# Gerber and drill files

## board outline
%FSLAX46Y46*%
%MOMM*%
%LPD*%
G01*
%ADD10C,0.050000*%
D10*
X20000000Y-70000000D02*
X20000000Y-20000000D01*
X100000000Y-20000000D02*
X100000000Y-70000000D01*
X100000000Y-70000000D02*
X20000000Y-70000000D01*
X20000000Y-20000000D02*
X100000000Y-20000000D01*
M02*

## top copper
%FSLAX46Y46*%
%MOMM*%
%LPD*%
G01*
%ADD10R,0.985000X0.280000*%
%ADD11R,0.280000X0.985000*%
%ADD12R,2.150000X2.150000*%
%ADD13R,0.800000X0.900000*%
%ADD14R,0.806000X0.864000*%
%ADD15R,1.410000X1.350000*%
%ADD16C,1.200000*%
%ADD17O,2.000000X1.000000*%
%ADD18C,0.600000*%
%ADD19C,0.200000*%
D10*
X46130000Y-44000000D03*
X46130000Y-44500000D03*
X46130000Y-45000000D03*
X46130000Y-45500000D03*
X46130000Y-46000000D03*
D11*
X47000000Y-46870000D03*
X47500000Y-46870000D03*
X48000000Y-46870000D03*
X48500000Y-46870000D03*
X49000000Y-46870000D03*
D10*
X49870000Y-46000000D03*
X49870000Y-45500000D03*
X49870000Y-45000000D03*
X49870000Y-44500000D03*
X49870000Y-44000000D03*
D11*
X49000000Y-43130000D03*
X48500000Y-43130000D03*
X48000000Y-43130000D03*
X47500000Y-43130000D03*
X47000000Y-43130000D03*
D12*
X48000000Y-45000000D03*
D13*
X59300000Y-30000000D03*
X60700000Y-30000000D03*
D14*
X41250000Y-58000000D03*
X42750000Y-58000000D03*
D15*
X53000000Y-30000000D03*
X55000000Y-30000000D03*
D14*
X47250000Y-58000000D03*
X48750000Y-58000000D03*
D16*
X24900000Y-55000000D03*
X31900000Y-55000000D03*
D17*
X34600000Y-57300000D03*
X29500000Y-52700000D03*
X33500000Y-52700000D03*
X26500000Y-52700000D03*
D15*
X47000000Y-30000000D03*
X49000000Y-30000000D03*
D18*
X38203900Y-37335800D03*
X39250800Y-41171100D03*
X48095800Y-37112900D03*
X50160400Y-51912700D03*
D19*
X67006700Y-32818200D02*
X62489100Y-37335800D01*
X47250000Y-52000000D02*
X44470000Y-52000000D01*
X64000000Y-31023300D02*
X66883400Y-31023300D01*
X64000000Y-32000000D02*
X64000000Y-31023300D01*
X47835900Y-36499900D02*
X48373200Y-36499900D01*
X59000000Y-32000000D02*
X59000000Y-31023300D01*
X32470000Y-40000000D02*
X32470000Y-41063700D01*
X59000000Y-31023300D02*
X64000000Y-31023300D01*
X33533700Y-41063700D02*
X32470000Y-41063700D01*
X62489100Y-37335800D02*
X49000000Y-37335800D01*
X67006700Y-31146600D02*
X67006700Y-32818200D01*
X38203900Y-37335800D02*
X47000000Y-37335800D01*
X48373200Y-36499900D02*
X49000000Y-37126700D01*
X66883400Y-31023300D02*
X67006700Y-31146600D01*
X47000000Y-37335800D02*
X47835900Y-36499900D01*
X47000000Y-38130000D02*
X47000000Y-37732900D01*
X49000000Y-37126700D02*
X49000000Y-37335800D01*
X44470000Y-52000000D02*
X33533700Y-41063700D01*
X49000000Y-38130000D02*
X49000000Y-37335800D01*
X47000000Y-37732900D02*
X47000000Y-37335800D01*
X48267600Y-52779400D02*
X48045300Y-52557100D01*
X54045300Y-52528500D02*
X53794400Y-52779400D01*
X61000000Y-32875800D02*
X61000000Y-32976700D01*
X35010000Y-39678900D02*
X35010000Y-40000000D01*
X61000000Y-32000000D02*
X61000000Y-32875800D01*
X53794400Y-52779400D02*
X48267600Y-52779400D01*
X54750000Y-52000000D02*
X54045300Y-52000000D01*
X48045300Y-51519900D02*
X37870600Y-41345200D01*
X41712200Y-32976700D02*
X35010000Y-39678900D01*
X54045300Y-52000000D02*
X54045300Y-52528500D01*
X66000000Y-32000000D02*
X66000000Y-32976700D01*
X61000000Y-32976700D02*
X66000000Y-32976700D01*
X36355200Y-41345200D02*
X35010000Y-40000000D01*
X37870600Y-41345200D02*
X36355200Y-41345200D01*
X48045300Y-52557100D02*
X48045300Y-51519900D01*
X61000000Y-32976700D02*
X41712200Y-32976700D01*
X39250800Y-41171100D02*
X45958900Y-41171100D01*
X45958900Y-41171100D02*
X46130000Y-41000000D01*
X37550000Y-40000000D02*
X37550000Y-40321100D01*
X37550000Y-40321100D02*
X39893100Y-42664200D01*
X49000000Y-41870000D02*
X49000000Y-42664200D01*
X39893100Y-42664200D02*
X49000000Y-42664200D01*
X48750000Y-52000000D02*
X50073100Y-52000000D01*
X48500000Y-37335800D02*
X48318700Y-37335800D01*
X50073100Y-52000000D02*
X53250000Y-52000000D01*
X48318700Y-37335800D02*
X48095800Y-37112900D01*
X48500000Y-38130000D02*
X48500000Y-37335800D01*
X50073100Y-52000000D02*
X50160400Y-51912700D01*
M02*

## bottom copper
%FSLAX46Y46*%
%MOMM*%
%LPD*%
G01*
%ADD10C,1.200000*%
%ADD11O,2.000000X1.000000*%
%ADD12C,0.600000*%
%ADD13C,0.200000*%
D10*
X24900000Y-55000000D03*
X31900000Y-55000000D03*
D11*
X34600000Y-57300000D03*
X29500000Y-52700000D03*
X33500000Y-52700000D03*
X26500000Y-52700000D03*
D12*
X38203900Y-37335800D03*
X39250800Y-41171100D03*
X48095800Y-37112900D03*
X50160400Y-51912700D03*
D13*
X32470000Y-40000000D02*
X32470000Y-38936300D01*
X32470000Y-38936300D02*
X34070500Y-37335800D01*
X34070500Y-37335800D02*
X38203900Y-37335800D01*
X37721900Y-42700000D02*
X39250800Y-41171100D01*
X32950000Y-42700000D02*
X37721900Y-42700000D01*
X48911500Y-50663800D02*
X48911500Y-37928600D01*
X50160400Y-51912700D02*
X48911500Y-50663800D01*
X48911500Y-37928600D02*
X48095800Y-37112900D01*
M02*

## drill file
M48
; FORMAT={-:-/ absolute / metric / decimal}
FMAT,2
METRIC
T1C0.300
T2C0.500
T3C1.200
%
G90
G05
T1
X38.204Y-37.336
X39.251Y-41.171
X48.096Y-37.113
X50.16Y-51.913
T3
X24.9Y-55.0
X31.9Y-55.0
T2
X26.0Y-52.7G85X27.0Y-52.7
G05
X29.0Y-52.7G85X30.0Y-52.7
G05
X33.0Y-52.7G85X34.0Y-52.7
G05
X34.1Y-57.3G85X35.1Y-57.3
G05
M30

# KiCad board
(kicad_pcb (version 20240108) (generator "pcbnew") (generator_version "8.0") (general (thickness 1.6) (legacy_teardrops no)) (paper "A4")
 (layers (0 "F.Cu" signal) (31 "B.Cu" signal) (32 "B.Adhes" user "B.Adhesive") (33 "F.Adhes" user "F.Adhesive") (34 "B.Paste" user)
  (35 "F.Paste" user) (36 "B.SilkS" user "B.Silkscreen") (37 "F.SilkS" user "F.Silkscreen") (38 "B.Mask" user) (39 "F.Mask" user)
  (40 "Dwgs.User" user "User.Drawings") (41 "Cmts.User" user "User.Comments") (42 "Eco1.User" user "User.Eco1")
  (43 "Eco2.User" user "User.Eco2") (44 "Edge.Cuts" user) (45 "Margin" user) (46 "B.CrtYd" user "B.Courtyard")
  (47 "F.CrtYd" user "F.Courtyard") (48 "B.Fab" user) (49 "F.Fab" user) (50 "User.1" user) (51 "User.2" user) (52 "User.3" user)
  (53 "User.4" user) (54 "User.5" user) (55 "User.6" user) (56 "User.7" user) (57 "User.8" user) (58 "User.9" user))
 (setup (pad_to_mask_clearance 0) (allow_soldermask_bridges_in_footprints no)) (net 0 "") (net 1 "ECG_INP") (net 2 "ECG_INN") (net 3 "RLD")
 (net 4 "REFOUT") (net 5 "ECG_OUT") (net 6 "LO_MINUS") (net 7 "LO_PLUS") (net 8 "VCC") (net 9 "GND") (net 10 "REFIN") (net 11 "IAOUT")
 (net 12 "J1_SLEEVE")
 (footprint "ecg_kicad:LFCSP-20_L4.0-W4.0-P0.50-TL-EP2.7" (layer "F.Cu") (at 48 45)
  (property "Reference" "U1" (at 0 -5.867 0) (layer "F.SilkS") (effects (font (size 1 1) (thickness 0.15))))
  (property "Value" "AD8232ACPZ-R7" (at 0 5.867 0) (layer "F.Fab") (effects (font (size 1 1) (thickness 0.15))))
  (pad "1" smd rect (at -1.87 -1) (size 0.985 0.28) (layers "F.Cu" "F.Paste" "F.Mask"))
  (pad "2" smd rect (at -1.87 -0.5) (size 0.985 0.28) (layers "F.Cu" "F.Paste" "F.Mask") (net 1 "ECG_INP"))
  (pad "3" smd rect (at -1.87 0) (size 0.985 0.28) (layers "F.Cu" "F.Paste" "F.Mask") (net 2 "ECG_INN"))
  (pad "4" smd rect (at -1.87 0.5) (size 0.985 0.28) (layers "F.Cu" "F.Paste" "F.Mask") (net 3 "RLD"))
  (pad "5" smd rect (at -1.87 1) (size 0.985 0.28) (layers "F.Cu" "F.Paste" "F.Mask") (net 3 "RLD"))
  (pad "6" smd rect (at -1 1.87) (size 0.28 0.985) (layers "F.Cu" "F.Paste" "F.Mask"))
  (pad "7" smd rect (at -0.5 1.87) (size 0.28 0.985) (layers "F.Cu" "F.Paste" "F.Mask"))
  (pad "8" smd rect (at 0 1.87) (size 0.28 0.985) (layers "F.Cu" "F.Paste" "F.Mask") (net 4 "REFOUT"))
  (pad "9" smd rect (at 0.5 1.87) (size 0.28 0.985) (layers "F.Cu" "F.Paste" "F.Mask"))
  (pad "10" smd rect (at 1 1.87) (size 0.28 0.985) (layers "F.Cu" "F.Paste" "F.Mask") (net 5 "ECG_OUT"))
  (pad "11" smd rect (at 1.87 1) (size 0.985 0.28) (layers "F.Cu" "F.Paste" "F.Mask") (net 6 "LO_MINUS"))
  (pad "12" smd rect (at 1.87 0.5) (size 0.985 0.28) (layers "F.Cu" "F.Paste" "F.Mask") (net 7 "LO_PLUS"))
  (pad "13" smd rect (at 1.87 0) (size 0.985 0.28) (layers "F.Cu" "F.Paste" "F.Mask") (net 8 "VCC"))
  (pad "14" smd rect (at 1.87 -0.5) (size 0.985 0.28) (layers "F.Cu" "F.Paste" "F.Mask") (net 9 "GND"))
  (pad "15" smd rect (at 1.87 -1) (size 0.985 0.28) (layers "F.Cu" "F.Paste" "F.Mask"))
  (pad "16" smd rect (at 1 -1.87) (size 0.28 0.985) (layers "F.Cu" "F.Paste" "F.Mask") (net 8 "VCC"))
  (pad "17" smd rect (at 0.5 -1.87) (size 0.28 0.985) (layers "F.Cu" "F.Paste" "F.Mask") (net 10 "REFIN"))
  (pad "18" smd rect (at 0 -1.87) (size 0.28 0.985) (layers "F.Cu" "F.Paste" "F.Mask") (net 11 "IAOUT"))
  (pad "19" smd rect (at -0.5 -1.87) (size 0.28 0.985) (layers "F.Cu" "F.Paste" "F.Mask"))
  (pad "20" smd rect (at -1 -1.87) (size 0.28 0.985) (layers "F.Cu" "F.Paste" "F.Mask") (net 8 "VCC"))
  (pad "21" smd rect (at 0 0) (size 2.15 2.15) (layers "F.Cu" "F.Paste" "F.Mask") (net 9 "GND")))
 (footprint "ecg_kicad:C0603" (layer "F.Cu") (at 60 30)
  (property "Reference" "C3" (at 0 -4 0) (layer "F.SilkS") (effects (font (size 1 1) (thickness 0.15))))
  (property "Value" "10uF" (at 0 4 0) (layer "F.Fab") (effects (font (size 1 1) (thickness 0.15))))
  (pad "1" smd rect (at -0.7 0) (size 0.8 0.9) (layers "F.Cu" "F.Paste" "F.Mask") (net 8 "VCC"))
  (pad "2" smd rect (at 0.7 0) (size 0.8 0.9) (layers "F.Cu" "F.Paste" "F.Mask") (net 9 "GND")))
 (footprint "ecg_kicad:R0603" (layer "F.Cu") (at 42 58)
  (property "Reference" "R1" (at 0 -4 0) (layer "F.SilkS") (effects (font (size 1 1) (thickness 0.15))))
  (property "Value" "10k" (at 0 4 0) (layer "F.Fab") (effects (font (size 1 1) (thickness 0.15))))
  (pad "1" smd rect (at -0.75 0) (size 0.806 0.864) (layers "F.Cu" "F.Paste" "F.Mask") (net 8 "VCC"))
  (pad "2" smd rect (at 0.75 0) (size 0.806 0.864) (layers "F.Cu" "F.Paste" "F.Mask") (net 10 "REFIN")))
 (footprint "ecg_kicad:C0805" (layer "F.Cu") (at 54 30)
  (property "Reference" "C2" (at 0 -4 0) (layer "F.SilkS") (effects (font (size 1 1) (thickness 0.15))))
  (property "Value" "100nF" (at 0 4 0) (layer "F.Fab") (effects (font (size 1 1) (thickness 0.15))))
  (pad "1" smd rect (at -1 0) (size 1.41 1.35) (layers "F.Cu" "F.Paste" "F.Mask") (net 8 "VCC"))
  (pad "2" smd rect (at 1 0) (size 1.41 1.35) (layers "F.Cu" "F.Paste" "F.Mask") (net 9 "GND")))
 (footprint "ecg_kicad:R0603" (layer "F.Cu") (at 48 58)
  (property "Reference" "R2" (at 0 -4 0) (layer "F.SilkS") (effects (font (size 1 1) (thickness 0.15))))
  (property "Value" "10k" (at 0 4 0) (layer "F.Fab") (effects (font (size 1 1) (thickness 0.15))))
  (pad "1" smd rect (at -0.75 0) (size 0.806 0.864) (layers "F.Cu" "F.Paste" "F.Mask") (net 10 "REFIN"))
  (pad "2" smd rect (at 0.75 0) (size 0.806 0.864) (layers "F.Cu" "F.Paste" "F.Mask") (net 9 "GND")))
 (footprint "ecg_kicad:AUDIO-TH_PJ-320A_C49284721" (layer "F.Cu") (at 30.55 55)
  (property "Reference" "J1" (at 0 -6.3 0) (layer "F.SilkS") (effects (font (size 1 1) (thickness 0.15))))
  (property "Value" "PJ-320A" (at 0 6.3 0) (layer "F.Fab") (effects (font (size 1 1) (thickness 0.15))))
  (pad "" thru_hole circle (at -5.65 0) (size 1.2 1.2) (drill 1.2) (layers "*.Cu" "*.Mask") (remove_unused_layers no))
  (pad "" thru_hole circle (at 1.35 0) (size 1.2 1.2) (drill 1.2) (layers "*.Cu" "*.Mask") (remove_unused_layers no))
  (pad "2" thru_hole oval (at 4.05 2.3 90) (size 1 2) (drill oval 0.500024 1.499997) (layers "*.Cu" "*.Mask") (remove_unused_layers no)
   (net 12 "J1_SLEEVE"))
  (pad "3" thru_hole oval (at -1.05 -2.3 90) (size 1 2) (drill oval 0.500024 1.499997) (layers "*.Cu" "*.Mask") (remove_unused_layers no)
   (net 2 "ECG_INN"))
  (pad "4" thru_hole oval (at 2.95 -2.3 90) (size 1 2) (drill oval 0.500024 1.499997) (layers "*.Cu" "*.Mask") (remove_unused_layers no)
   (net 3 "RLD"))
  (pad "5" thru_hole oval (at -4.05 -2.3 90) (size 1 2) (drill oval 0.500024 1.499997) (layers "*.Cu" "*.Mask") (remove_unused_layers no)
   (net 1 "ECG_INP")))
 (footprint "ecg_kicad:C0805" (layer "F.Cu") (at 48 30)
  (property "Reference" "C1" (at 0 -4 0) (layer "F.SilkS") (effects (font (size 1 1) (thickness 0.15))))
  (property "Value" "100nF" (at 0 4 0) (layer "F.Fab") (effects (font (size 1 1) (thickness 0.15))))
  (pad "1" smd rect (at -1 0) (size 1.41 1.35) (layers "F.Cu" "F.Paste" "F.Mask") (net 8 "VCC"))
  (pad "2" smd rect (at 1 0) (size 1.41 1.35) (layers "F.Cu" "F.Paste" "F.Mask") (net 9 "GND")))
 (gr_line (start 20 70) (end 20 20) (stroke (width 0.05) (type default)) (layer "Edge.Cuts"))
 (gr_line (start 100 20) (end 100 70) (stroke (width 0.05) (type default)) (layer "Edge.Cuts"))
 (gr_line (start 100 70) (end 20 70) (stroke (width 0.05) (type default)) (layer "Edge.Cuts"))
 (gr_line (start 20 20) (end 100 20) (stroke (width 0.05) (type default)) (layer "Edge.Cuts"))
 (segment (start 67.0067 32.8182) (end 62.4891 37.3358) (width 0.2) (layer "F.Cu") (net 8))
 (segment (start 47.25 52) (end 44.47 52) (width 0.2) (layer "F.Cu") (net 8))
 (segment (start 64 31.0233) (end 66.8834 31.0233) (width 0.2) (layer "F.Cu") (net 8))
 (segment (start 64 32) (end 64 31.0233) (width 0.2) (layer "F.Cu") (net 8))
 (segment (start 47.8359 36.4999) (end 48.3732 36.4999) (width 0.2) (layer "F.Cu") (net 8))
 (segment (start 59 32) (end 59 31.0233) (width 0.2) (layer "F.Cu") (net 8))
 (segment (start 32.47 40) (end 32.47 41.0637) (width 0.2) (layer "F.Cu") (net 8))
 (segment (start 59 31.0233) (end 64 31.0233) (width 0.2) (layer "F.Cu") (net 8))
 (segment (start 33.5337 41.0637) (end 32.47 41.0637) (width 0.2) (layer "F.Cu") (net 8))
 (segment (start 62.4891 37.3358) (end 49 37.3358) (width 0.2) (layer "F.Cu") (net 8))
 (segment (start 67.0067 31.1466) (end 67.0067 32.8182) (width 0.2) (layer "F.Cu") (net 8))
 (segment (start 38.2039 37.3358) (end 47 37.3358) (width 0.2) (layer "F.Cu") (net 8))
 (segment (start 48.3732 36.4999) (end 49 37.1267) (width 0.2) (layer "F.Cu") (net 8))
 (segment (start 66.8834 31.0233) (end 67.0067 31.1466) (width 0.2) (layer "F.Cu") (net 8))
 (segment (start 47 37.3358) (end 47.8359 36.4999) (width 0.2) (layer "F.Cu") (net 8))
 (segment (start 47 38.13) (end 47 37.7329) (width 0.2) (layer "F.Cu") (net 8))
 (segment (start 49 37.1267) (end 49 37.3358) (width 0.2) (layer "F.Cu") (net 8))
 (segment (start 44.47 52) (end 33.5337 41.0637) (width 0.2) (layer "F.Cu") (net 8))
 (segment (start 49 38.13) (end 49 37.3358) (width 0.2) (layer "F.Cu") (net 8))
 (segment (start 47 37.7329) (end 47 37.3358) (width 0.2) (layer "F.Cu") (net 8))
 (via (at 38.2039 37.3358) (size 0.6) (drill 0.3) (layers "F.Cu" "B.Cu") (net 8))
 (segment (start 32.47 40) (end 32.47 38.9363) (width 0.2) (layer "B.Cu") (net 8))
 (segment (start 32.47 38.9363) (end 34.0705 37.3358) (width 0.2) (layer "B.Cu") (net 8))
 (segment (start 34.0705 37.3358) (end 38.2039 37.3358) (width 0.2) (layer "B.Cu") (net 8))
 (segment (start 48.2676 52.7794) (end 48.0453 52.5571) (width 0.2) (layer "F.Cu") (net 9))
 (segment (start 54.0453 52.5285) (end 53.7944 52.7794) (width 0.2) (layer "F.Cu") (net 9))
 (segment (start 61 32.8758) (end 61 32.9767) (width 0.2) (layer "F.Cu") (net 9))
 (segment (start 35.01 39.6789) (end 35.01 40) (width 0.2) (layer "F.Cu") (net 9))
 (segment (start 61 32) (end 61 32.8758) (width 0.2) (layer "F.Cu") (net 9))
 (segment (start 53.7944 52.7794) (end 48.2676 52.7794) (width 0.2) (layer "F.Cu") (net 9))
 (segment (start 54.75 52) (end 54.0453 52) (width 0.2) (layer "F.Cu") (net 9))
 (segment (start 48.0453 51.5199) (end 37.8706 41.3452) (width 0.2) (layer "F.Cu") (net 9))
 (segment (start 41.7122 32.9767) (end 35.01 39.6789) (width 0.2) (layer "F.Cu") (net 9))
 (segment (start 54.0453 52) (end 54.0453 52.5285) (width 0.2) (layer "F.Cu") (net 9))
 (segment (start 66 32) (end 66 32.9767) (width 0.2) (layer "F.Cu") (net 9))
 (segment (start 61 32.9767) (end 66 32.9767) (width 0.2) (layer "F.Cu") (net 9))
 (segment (start 36.3552 41.3452) (end 35.01 40) (width 0.2) (layer "F.Cu") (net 9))
 (segment (start 37.8706 41.3452) (end 36.3552 41.3452) (width 0.2) (layer "F.Cu") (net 9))
 (segment (start 48.0453 52.5571) (end 48.0453 51.5199) (width 0.2) (layer "F.Cu") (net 9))
 (segment (start 61 32.9767) (end 41.7122 32.9767) (width 0.2) (layer "F.Cu") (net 9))
 (segment (start 39.2508 41.1711) (end 45.9589 41.1711) (width 0.2) (layer "F.Cu") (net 3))
 (segment (start 45.9589 41.1711) (end 46.13 41) (width 0.2) (layer "F.Cu") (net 3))
 (via (at 39.2508 41.1711) (size 0.6) (drill 0.3) (layers "F.Cu" "B.Cu") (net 3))
 (segment (start 37.7219 42.7) (end 39.2508 41.1711) (width 0.2) (layer "B.Cu") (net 3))
 (segment (start 32.95 42.7) (end 37.7219 42.7) (width 0.2) (layer "B.Cu") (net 3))
 (segment (start 37.55 40) (end 37.55 40.3211) (width 0.2) (layer "F.Cu") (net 5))
 (segment (start 37.55 40.3211) (end 39.8931 42.6642) (width 0.2) (layer "F.Cu") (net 5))
 (segment (start 49 41.87) (end 49 42.6642) (width 0.2) (layer "F.Cu") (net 5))
 (segment (start 39.8931 42.6642) (end 49 42.6642) (width 0.2) (layer "F.Cu") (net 5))
 (segment (start 48.75 52) (end 50.0731 52) (width 0.2) (layer "F.Cu") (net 6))
 (segment (start 48.5 37.3358) (end 48.3187 37.3358) (width 0.2) (layer "F.Cu") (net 6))
 (segment (start 50.0731 52) (end 53.25 52) (width 0.2) (layer "F.Cu") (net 6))
 (segment (start 48.3187 37.3358) (end 48.0958 37.1129) (width 0.2) (layer "F.Cu") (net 6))
 (segment (start 48.5 38.13) (end 48.5 37.3358) (width 0.2) (layer "F.Cu") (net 6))
 (segment (start 50.0731 52) (end 50.1604 51.9127) (width 0.2) (layer "F.Cu") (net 6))
 (via (at 48.0958 37.1129) (size 0.6) (drill 0.3) (layers "F.Cu" "B.Cu") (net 6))
 (via (at 50.1604 51.9127) (size 0.6) (drill 0.3) (layers "F.Cu" "B.Cu") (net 6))
 (segment (start 48.9115 50.6638) (end 48.9115 37.9286) (width 0.2) (layer "B.Cu") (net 6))
 (segment (start 50.1604 51.9127) (end 48.9115 50.6638) (width 0.2) (layer "B.Cu") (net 6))
 (segment (start 48.9115 37.9286) (end 48.0958 37.1129) (width 0.2) (layer "B.Cu") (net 6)))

